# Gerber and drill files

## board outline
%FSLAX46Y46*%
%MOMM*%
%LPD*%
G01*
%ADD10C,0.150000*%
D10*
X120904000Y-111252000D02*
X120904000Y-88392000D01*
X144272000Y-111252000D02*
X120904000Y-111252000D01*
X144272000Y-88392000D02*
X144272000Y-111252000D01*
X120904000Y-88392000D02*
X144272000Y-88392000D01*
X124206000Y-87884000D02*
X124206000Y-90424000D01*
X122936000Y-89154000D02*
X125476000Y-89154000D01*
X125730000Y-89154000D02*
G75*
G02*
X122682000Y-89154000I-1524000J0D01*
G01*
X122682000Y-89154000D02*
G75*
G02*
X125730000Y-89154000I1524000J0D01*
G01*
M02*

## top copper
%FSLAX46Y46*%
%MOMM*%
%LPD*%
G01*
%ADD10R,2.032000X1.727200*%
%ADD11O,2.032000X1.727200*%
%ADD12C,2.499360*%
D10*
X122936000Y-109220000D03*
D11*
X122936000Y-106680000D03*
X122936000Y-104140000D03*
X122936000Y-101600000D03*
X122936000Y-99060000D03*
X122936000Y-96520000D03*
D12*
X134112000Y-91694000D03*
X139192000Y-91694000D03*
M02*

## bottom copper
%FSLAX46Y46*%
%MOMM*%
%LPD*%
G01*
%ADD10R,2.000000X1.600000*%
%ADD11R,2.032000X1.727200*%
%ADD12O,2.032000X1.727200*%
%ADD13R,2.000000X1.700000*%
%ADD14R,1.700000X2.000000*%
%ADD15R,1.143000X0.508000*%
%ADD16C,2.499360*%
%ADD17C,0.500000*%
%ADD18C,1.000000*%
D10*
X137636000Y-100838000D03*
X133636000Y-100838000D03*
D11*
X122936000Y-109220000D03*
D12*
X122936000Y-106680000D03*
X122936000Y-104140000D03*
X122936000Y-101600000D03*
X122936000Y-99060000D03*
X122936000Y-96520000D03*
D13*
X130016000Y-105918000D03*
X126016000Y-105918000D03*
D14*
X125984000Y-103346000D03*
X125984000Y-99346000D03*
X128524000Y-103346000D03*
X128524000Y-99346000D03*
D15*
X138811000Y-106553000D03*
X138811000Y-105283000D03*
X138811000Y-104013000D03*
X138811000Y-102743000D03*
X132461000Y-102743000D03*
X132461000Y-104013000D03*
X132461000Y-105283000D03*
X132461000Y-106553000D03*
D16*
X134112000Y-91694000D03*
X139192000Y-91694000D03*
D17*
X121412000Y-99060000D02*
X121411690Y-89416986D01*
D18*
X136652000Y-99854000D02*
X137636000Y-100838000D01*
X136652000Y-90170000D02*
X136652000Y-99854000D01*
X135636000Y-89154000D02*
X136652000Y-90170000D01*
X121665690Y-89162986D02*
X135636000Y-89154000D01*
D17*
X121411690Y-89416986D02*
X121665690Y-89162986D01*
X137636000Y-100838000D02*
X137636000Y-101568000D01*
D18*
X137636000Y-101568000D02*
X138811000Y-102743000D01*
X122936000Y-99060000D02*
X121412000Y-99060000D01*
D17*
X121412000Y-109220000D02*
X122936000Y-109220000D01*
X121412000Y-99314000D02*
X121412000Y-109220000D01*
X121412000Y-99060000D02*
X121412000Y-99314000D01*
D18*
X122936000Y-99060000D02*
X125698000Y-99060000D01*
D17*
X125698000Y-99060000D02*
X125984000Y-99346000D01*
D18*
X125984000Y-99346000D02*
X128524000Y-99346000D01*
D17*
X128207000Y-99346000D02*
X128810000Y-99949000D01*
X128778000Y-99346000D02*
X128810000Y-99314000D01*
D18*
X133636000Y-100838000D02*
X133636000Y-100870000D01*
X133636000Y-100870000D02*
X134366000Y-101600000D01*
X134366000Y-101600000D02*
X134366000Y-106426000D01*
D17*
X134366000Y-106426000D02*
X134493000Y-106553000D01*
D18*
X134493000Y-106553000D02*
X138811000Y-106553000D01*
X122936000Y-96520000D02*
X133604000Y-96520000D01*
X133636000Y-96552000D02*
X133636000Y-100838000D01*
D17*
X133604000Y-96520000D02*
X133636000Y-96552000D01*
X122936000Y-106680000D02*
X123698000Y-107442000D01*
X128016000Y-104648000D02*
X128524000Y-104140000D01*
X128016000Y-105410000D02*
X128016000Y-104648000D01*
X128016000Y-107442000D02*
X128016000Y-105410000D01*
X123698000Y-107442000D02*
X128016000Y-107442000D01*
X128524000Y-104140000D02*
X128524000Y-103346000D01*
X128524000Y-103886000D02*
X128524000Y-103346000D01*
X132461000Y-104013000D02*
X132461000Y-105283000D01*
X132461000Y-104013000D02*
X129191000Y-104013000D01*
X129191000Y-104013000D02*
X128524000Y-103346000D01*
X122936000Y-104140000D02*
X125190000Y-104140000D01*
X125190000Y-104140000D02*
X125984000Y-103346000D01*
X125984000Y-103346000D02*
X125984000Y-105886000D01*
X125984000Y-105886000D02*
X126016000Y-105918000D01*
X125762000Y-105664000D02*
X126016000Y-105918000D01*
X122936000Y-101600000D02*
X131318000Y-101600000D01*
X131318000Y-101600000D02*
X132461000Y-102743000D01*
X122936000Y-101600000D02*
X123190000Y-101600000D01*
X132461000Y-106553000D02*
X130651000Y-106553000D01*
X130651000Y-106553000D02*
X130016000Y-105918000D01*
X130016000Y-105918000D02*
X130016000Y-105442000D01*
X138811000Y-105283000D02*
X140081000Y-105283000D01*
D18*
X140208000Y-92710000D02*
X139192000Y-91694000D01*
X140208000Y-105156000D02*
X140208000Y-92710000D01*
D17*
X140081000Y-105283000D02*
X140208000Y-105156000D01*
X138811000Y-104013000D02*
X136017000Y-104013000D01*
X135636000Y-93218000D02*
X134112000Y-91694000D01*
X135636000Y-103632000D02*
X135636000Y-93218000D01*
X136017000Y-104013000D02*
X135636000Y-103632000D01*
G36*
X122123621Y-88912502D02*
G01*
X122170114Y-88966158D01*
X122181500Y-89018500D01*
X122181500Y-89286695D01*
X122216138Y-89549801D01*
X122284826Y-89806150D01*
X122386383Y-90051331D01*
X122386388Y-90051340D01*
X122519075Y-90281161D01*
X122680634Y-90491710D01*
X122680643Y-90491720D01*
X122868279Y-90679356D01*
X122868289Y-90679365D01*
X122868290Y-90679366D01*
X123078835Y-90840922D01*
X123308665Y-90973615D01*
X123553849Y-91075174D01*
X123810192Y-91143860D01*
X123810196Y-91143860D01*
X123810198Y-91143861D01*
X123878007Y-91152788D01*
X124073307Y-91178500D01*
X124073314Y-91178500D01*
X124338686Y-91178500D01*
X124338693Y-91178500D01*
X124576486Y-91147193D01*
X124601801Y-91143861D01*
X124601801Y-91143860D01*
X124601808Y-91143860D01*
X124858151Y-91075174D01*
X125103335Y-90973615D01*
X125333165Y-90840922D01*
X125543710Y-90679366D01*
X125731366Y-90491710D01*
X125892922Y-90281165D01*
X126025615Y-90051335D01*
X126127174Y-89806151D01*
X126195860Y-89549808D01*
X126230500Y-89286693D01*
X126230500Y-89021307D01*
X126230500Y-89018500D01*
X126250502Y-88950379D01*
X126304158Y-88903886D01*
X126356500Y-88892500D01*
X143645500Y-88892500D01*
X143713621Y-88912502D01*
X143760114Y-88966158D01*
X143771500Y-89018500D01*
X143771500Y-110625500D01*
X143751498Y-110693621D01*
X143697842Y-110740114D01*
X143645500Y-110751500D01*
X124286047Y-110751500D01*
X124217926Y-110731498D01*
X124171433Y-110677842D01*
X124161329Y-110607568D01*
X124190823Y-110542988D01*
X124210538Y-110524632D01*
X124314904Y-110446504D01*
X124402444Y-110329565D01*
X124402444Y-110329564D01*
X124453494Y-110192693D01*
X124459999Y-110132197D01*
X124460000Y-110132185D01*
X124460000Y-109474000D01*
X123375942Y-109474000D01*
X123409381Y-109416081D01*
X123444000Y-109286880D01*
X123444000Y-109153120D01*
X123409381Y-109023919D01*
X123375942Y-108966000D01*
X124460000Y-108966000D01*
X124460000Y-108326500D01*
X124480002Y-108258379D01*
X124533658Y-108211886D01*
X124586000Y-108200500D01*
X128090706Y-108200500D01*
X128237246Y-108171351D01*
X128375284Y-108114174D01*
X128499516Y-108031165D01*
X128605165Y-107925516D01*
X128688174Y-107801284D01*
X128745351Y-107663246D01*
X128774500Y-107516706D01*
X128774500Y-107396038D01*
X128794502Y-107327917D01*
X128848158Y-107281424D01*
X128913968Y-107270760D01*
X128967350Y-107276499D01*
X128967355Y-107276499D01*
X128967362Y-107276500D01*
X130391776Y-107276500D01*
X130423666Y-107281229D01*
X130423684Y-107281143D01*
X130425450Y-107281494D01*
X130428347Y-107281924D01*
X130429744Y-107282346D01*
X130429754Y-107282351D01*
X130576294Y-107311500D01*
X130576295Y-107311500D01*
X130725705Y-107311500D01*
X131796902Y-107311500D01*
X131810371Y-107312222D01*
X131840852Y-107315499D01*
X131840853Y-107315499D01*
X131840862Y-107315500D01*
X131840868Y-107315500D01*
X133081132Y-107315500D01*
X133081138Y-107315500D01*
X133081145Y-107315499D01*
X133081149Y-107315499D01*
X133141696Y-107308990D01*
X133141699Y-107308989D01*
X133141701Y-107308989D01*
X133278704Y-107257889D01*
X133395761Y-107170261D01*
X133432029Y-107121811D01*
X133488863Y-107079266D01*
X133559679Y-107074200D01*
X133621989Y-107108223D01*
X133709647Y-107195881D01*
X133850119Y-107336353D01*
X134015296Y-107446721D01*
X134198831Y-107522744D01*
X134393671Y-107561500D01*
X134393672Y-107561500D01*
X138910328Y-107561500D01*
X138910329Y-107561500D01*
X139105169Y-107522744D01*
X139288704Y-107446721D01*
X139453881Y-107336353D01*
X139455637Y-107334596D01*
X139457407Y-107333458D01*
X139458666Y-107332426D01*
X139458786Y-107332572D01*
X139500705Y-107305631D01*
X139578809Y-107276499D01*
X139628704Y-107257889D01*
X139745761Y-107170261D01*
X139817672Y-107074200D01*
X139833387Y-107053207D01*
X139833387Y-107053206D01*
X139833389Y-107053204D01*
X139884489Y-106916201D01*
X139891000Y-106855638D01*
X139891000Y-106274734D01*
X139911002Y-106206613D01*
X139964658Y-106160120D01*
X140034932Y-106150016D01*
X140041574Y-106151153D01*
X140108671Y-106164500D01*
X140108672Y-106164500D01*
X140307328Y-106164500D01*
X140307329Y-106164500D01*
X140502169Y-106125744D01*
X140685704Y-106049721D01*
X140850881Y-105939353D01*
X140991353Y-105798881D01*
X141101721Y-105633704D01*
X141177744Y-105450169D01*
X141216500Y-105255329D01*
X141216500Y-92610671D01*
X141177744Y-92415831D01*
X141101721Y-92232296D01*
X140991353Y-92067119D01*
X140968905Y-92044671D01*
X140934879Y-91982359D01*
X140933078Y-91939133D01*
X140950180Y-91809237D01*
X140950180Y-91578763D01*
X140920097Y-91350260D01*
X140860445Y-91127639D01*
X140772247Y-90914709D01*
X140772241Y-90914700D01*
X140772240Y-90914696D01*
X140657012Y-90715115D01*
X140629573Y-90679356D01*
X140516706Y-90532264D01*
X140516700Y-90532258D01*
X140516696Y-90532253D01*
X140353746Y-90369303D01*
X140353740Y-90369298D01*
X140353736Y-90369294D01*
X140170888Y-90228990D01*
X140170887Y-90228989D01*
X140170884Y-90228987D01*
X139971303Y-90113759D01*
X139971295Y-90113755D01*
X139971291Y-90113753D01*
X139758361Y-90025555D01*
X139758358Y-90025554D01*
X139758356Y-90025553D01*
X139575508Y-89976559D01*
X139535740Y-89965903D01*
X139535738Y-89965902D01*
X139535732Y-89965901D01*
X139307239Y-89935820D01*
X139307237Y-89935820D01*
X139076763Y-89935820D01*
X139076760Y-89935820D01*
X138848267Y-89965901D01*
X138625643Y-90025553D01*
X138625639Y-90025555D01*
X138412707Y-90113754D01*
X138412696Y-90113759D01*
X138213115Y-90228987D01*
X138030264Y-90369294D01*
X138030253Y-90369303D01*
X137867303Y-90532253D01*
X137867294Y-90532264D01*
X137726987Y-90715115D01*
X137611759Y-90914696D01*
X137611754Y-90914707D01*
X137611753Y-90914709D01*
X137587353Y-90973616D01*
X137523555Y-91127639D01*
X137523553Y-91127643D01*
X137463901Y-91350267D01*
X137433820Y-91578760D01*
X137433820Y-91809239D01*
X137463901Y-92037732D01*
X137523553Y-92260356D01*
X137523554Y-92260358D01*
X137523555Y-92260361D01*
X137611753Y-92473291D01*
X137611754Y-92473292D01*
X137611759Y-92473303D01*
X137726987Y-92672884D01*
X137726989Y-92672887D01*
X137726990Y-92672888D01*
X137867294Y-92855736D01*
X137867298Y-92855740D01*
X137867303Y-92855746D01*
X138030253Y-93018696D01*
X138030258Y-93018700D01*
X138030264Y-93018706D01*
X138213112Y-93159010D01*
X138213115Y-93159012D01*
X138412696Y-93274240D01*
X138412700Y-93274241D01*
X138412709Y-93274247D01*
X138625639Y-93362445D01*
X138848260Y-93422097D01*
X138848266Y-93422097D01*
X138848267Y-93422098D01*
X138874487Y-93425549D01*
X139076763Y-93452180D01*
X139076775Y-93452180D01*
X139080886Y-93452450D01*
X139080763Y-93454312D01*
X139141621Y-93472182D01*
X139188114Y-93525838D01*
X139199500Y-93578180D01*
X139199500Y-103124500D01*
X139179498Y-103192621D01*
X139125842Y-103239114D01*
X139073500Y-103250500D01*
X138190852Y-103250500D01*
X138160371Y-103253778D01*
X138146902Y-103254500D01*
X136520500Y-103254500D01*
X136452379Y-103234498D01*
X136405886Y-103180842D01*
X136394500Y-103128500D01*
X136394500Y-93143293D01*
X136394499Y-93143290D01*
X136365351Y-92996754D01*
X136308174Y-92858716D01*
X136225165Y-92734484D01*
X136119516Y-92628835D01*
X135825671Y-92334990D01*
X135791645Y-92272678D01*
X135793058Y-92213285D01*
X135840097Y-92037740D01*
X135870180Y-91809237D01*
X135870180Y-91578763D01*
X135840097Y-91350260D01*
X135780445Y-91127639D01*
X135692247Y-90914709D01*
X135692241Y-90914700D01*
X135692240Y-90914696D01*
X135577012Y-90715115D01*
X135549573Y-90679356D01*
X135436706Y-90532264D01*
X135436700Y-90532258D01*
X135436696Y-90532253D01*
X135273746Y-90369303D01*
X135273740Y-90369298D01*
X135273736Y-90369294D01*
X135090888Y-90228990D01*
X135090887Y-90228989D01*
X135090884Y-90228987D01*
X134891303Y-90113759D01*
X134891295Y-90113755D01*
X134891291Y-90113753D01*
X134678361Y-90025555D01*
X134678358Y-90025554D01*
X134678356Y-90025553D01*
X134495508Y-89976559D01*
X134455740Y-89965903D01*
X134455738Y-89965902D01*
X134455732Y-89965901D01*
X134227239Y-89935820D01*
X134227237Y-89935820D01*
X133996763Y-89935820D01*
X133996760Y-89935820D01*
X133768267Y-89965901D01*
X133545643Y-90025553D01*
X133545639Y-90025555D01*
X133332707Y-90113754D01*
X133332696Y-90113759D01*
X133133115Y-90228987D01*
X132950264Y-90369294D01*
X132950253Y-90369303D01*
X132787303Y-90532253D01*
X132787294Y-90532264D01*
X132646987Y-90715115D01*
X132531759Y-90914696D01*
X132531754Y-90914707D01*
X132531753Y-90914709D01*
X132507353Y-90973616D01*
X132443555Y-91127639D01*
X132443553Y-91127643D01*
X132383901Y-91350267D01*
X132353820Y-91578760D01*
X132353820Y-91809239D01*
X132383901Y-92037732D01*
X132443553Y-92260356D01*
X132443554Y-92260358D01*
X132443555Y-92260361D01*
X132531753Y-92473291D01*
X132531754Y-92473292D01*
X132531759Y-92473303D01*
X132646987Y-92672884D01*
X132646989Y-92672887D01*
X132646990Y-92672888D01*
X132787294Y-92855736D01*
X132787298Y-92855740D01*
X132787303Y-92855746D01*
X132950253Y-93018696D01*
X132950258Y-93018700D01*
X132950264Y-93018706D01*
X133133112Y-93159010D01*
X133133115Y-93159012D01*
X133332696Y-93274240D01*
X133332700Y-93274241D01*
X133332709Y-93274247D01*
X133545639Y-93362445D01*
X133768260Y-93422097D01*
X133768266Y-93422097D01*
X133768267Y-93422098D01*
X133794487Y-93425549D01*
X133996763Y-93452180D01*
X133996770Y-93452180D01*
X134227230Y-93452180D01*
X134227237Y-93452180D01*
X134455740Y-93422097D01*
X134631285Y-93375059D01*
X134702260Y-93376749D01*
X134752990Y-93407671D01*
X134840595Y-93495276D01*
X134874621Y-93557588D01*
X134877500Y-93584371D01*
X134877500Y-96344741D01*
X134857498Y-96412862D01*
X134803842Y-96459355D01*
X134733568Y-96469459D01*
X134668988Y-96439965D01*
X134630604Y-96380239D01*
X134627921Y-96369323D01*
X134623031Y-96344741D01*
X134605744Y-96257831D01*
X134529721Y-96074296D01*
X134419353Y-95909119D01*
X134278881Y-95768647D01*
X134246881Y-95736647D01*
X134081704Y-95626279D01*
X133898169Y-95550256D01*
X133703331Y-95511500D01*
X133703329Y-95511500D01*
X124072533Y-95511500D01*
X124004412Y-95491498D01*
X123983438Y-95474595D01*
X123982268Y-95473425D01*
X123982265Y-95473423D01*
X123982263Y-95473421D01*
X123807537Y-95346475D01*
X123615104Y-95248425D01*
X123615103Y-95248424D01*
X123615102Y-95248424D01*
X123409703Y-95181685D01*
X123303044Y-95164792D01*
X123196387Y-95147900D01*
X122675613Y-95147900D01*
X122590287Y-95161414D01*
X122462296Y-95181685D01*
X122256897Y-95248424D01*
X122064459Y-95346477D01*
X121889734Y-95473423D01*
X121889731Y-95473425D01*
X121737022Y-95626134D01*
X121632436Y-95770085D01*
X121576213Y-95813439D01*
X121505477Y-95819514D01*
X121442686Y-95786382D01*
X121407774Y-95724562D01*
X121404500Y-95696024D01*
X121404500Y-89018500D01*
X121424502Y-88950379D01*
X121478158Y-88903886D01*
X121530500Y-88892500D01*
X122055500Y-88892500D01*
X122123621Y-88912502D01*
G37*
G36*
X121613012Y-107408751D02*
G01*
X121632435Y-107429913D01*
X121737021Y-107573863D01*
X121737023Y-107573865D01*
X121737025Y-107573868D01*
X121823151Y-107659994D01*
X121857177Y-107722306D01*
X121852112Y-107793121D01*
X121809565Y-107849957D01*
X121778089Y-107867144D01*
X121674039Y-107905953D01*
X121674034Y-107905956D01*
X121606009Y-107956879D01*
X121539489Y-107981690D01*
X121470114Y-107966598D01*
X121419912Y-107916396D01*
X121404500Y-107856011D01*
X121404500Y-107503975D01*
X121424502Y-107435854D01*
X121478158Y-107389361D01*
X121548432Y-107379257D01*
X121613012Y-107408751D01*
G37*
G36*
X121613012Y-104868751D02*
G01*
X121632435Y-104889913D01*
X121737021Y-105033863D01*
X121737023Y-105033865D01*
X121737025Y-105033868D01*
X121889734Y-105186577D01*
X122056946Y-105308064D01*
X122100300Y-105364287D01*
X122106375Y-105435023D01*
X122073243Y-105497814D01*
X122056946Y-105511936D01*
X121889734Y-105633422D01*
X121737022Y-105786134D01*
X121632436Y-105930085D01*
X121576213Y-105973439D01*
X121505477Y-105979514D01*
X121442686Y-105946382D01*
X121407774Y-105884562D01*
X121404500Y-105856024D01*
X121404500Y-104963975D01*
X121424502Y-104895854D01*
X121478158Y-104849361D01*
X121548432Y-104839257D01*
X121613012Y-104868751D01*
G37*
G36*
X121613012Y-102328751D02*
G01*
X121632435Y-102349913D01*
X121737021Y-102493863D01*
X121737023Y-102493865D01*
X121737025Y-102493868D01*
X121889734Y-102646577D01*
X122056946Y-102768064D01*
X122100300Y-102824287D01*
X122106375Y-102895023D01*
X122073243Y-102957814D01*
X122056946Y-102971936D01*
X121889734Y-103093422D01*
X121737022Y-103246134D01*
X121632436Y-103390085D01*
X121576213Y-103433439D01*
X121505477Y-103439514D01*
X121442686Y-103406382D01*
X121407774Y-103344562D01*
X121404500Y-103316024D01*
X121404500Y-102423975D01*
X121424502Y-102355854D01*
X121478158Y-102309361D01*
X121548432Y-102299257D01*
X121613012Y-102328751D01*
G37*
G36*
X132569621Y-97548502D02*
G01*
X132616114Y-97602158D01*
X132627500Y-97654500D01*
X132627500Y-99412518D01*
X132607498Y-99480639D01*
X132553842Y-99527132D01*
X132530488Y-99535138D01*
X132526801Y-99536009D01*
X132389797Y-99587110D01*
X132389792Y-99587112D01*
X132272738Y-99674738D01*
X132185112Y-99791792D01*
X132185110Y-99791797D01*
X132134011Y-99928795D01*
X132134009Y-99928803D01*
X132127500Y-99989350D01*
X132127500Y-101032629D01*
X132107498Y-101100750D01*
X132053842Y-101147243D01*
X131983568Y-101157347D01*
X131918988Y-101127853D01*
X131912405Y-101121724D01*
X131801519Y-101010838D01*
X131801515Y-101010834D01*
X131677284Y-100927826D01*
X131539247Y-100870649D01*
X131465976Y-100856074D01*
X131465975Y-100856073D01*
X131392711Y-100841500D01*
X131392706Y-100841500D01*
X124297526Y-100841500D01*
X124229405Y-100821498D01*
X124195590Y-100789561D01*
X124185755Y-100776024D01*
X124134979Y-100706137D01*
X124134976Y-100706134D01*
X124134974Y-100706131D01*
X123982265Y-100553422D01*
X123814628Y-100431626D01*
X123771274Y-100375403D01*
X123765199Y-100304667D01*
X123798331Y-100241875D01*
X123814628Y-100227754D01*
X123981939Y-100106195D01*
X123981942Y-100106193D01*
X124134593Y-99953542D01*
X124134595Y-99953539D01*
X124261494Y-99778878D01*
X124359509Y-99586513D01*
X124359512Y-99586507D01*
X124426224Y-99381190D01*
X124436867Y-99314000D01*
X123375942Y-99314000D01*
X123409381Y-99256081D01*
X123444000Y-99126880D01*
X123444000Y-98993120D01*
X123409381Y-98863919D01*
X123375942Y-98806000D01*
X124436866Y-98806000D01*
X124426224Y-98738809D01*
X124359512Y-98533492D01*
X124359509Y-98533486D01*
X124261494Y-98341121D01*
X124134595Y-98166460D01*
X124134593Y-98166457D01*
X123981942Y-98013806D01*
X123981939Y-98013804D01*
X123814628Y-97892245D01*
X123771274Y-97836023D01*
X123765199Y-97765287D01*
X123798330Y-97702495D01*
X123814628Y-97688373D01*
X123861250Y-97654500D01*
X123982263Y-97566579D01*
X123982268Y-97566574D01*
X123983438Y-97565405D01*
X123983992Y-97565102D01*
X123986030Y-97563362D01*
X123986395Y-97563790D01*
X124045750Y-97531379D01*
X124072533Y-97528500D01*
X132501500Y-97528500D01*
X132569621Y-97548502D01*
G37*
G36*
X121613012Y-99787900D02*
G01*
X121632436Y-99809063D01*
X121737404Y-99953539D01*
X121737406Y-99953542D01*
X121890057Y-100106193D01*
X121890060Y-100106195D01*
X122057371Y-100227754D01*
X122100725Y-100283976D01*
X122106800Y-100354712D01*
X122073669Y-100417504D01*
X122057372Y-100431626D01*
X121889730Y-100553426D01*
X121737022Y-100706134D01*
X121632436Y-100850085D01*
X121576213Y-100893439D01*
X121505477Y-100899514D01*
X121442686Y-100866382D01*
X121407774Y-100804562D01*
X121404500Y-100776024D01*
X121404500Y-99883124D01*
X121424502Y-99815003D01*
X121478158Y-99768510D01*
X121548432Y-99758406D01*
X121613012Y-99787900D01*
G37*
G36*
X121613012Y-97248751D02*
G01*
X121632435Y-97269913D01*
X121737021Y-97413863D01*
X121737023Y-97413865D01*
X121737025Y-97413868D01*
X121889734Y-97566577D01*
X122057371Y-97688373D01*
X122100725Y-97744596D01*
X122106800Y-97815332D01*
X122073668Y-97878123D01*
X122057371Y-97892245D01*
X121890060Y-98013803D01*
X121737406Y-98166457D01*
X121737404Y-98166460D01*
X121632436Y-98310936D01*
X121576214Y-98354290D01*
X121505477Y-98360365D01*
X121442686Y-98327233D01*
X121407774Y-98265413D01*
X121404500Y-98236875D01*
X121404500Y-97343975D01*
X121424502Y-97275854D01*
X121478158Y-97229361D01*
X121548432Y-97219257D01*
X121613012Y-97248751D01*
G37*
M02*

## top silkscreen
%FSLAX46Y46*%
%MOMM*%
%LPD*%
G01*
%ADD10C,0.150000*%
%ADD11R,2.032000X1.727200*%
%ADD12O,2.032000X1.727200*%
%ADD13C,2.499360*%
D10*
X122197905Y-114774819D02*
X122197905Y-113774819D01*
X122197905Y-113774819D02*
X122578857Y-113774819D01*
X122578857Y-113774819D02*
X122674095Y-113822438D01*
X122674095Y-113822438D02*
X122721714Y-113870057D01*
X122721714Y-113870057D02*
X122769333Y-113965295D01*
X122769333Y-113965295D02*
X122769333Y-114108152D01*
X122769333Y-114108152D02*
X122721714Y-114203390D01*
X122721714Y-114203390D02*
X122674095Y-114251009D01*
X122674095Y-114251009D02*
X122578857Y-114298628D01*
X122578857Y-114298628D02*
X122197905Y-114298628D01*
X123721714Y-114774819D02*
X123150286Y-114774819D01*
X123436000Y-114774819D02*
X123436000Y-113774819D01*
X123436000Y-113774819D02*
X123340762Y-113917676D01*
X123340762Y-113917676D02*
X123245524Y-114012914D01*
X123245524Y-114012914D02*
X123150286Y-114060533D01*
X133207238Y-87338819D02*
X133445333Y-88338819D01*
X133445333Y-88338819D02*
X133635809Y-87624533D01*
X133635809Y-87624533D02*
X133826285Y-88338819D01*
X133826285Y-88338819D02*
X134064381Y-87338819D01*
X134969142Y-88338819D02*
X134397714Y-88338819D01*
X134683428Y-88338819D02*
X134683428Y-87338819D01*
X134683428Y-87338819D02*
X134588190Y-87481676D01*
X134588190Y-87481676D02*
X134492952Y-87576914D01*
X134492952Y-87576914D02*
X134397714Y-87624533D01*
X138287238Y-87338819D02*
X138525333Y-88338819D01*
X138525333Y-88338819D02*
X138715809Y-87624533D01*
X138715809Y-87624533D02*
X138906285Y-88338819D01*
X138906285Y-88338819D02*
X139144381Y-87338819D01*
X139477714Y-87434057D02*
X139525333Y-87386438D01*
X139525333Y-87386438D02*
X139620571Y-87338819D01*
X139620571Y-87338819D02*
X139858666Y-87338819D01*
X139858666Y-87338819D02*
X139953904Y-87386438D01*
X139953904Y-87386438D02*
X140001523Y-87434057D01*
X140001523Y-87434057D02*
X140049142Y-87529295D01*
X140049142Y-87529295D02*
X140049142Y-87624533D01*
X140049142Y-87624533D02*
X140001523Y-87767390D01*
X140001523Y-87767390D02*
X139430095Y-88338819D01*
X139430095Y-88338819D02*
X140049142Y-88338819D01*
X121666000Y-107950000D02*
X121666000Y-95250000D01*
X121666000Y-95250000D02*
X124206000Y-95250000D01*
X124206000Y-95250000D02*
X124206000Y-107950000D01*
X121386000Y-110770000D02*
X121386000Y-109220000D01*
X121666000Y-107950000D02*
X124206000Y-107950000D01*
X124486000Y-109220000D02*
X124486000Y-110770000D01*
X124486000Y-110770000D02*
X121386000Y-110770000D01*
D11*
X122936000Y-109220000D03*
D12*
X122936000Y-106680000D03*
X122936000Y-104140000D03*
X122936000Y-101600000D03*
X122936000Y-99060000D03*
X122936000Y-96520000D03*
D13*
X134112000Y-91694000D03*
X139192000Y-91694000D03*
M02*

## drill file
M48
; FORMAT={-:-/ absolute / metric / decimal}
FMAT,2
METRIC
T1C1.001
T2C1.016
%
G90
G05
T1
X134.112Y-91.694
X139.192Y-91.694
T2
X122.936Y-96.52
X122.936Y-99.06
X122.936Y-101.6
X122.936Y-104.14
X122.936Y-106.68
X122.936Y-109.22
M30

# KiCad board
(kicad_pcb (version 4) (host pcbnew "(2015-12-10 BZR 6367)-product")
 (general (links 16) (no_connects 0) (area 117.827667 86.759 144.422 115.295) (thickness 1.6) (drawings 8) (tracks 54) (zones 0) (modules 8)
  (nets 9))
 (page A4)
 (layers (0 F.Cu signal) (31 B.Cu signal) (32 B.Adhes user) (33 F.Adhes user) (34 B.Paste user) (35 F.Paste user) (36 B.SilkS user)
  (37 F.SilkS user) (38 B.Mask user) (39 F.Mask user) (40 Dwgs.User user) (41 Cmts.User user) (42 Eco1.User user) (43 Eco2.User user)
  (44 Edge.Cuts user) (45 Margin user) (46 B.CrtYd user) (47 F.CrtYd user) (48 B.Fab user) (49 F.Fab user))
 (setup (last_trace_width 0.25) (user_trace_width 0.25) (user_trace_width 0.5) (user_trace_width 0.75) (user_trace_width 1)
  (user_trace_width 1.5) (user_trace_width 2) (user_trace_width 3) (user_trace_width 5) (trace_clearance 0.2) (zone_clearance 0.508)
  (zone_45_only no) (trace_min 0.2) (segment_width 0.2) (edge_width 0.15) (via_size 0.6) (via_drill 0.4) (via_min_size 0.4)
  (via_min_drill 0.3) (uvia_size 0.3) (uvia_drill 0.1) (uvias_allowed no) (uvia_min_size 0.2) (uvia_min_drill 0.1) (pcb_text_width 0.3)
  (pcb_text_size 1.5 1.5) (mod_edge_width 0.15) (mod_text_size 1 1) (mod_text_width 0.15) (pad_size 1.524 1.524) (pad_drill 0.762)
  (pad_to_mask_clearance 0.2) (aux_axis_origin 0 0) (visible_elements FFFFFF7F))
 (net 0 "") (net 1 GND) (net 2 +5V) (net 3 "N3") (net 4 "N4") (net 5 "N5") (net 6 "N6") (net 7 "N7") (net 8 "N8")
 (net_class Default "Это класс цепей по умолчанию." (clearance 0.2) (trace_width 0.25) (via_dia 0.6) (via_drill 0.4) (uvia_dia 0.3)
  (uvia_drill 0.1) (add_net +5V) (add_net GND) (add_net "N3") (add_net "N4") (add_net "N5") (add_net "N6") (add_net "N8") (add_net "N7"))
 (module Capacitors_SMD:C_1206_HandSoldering (layer B.Cu) (at 135.636 100.838 180)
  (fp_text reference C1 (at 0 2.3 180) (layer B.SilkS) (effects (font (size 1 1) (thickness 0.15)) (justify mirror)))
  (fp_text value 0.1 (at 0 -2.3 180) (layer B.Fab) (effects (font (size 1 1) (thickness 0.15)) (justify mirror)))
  (pad 1 smd rect (at -2 0 180) (size 2 1.6) (layers B.Cu B.Paste B.Mask) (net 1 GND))
  (pad 2 smd rect (at 2 0 180) (size 2 1.6) (layers B.Cu B.Paste B.Mask) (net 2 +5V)))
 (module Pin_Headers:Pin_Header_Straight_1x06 (layer F.Cu) (at 122.936 109.22 180)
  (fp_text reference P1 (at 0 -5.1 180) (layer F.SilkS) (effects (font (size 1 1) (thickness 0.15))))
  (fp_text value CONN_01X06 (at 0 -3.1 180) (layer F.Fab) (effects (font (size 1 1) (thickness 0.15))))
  (fp_line (start 1.27 1.27) (end 1.27 13.97) (layer F.SilkS) (width 0.15))
  (fp_line (start 1.27 13.97) (end -1.27 13.97) (layer F.SilkS) (width 0.15))
  (fp_line (start -1.27 13.97) (end -1.27 1.27) (layer F.SilkS) (width 0.15))
  (fp_line (start 1.55 -1.55) (end 1.55 0) (layer F.SilkS) (width 0.15))
  (fp_line (start 1.27 1.27) (end -1.27 1.27) (layer F.SilkS) (width 0.15))
  (fp_line (start -1.55 0) (end -1.55 -1.55) (layer F.SilkS) (width 0.15))
  (fp_line (start -1.55 -1.55) (end 1.55 -1.55) (layer F.SilkS) (width 0.15))
  (pad 1 thru_hole rect (at 0 0 180) (size 2.032 1.7272) (drill 1.016) (layers *.Cu *.Mask F.SilkS) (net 1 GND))
  (pad 2 thru_hole oval (at 0 2.54 180) (size 2.032 1.7272) (drill 1.016) (layers *.Cu *.Mask F.SilkS) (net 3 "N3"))
  (pad 3 thru_hole oval (at 0 5.08 180) (size 2.032 1.7272) (drill 1.016) (layers *.Cu *.Mask F.SilkS) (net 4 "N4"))
  (pad 4 thru_hole oval (at 0 7.62 180) (size 2.032 1.7272) (drill 1.016) (layers *.Cu *.Mask F.SilkS) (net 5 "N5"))
  (pad 5 thru_hole oval (at 0 10.16 180) (size 2.032 1.7272) (drill 1.016) (layers *.Cu *.Mask F.SilkS) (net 1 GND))
  (pad 6 thru_hole oval (at 0 12.7 180) (size 2.032 1.7272) (drill 1.016) (layers *.Cu *.Mask F.SilkS) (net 2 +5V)))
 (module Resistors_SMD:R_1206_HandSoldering (layer B.Cu) (at 128.016 105.918 180)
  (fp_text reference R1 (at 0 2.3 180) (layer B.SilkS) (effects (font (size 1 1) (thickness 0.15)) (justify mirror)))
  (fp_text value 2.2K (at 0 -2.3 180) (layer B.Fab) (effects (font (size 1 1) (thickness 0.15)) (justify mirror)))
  (pad 1 smd rect (at -2 0 180) (size 2 1.7) (layers B.Cu B.Paste B.Mask) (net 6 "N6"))
  (pad 2 smd rect (at 2 0 180) (size 2 1.7) (layers B.Cu B.Paste B.Mask) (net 4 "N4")))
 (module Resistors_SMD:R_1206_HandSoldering (layer B.Cu) (at 125.984 101.346 90)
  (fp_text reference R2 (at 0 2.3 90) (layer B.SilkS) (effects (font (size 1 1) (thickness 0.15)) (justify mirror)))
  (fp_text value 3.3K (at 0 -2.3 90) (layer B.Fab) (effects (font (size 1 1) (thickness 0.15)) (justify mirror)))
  (pad 1 smd rect (at -2 0 90) (size 2 1.7) (layers B.Cu B.Paste B.Mask) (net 4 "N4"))
  (pad 2 smd rect (at 2 0 90) (size 2 1.7) (layers B.Cu B.Paste B.Mask) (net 1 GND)))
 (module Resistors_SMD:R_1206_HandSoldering (layer B.Cu) (at 128.524 101.346 90)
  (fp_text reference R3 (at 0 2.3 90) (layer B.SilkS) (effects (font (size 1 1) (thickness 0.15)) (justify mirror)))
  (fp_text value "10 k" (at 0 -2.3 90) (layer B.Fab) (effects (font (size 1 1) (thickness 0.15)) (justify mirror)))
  (pad 1 smd rect (at -2 0 90) (size 2 1.7) (layers B.Cu B.Paste B.Mask) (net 3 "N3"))
  (pad 2 smd rect (at 2 0 90) (size 2 1.7) (layers B.Cu B.Paste B.Mask) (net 1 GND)))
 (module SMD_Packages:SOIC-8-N (layer B.Cu) (at 135.636 104.648 90)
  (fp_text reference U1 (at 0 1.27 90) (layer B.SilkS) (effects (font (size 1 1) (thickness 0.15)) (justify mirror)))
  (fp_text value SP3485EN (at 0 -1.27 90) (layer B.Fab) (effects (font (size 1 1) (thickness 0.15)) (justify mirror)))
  (pad 8 smd rect (at -1.905 3.175 90) (size 0.508 1.143) (layers B.Cu B.Paste B.Mask) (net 2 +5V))
  (pad 7 smd rect (at -0.635 3.175 90) (size 0.508 1.143) (layers B.Cu B.Paste B.Mask) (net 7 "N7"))
  (pad 6 smd rect (at 0.635 3.175 90) (size 0.508 1.143) (layers B.Cu B.Paste B.Mask) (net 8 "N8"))
  (pad 5 smd rect (at 1.905 3.175 90) (size 0.508 1.143) (layers B.Cu B.Paste B.Mask) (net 1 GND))
  (pad 4 smd rect (at 1.905 -3.175 90) (size 0.508 1.143) (layers B.Cu B.Paste B.Mask) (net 5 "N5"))
  (pad 3 smd rect (at 0.635 -3.175 90) (size 0.508 1.143) (layers B.Cu B.Paste B.Mask) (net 3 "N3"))
  (pad 2 smd rect (at -0.635 -3.175 90) (size 0.508 1.143) (layers B.Cu B.Paste B.Mask) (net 3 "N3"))
  (pad 1 smd rect (at -1.905 -3.175 90) (size 0.508 1.143) (layers B.Cu B.Paste B.Mask) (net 6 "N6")))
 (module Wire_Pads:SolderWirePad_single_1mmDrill (layer F.Cu) (at 134.112 91.694)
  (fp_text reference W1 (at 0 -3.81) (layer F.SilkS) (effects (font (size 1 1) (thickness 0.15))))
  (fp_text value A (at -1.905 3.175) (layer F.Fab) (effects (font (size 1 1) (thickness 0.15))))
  (pad 1 thru_hole circle (at 0 0) (size 2.49936 2.49936) (drill 1.00076) (layers *.Cu *.Mask F.SilkS) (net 8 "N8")))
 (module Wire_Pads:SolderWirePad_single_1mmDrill (layer F.Cu) (at 139.192 91.694)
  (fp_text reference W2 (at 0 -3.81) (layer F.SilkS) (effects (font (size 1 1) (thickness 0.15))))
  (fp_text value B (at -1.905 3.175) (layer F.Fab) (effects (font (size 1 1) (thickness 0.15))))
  (pad 1 thru_hole circle (at 0 0) (size 2.49936 2.49936) (drill 1.00076) (layers *.Cu *.Mask F.SilkS) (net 7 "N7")))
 (gr_line (start 120.904 111.252) (end 120.904 88.392) (angle 90) (layer Edge.Cuts) (width 0.15))
 (gr_line (start 144.272 111.252) (end 120.904 111.252) (angle 90) (layer Edge.Cuts) (width 0.15))
 (gr_line (start 144.272 88.392) (end 144.272 111.252) (angle 90) (layer Edge.Cuts) (width 0.15))
 (gr_line (start 120.904 88.392) (end 144.272 88.392) (angle 90) (layer Edge.Cuts) (width 0.15))
 (gr_line (start 124.206 87.884) (end 124.206 90.424) (angle 90) (layer Edge.Cuts) (width 0.15))
 (gr_line (start 122.936 89.154) (end 125.476 89.154) (angle 90) (layer Edge.Cuts) (width 0.15))
 (gr_circle (center 124.206 89.154) (end 125.73 89.154) (layer Edge.Cuts) (width 0.15))
 (segment (start 121.412 99.06) (end 121.41169 89.416986) (width 0.5) (layer B.Cu) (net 1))
 (segment (start 136.652 99.854) (end 137.636 100.838) (width 1) (layer B.Cu) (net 1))
 (segment (start 136.652 90.17) (end 136.652 99.854) (width 1) (layer B.Cu) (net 1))
 (segment (start 135.636 89.154) (end 136.652 90.17) (width 1) (layer B.Cu) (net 1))
 (segment (start 121.66569 89.162986) (end 135.636 89.154) (width 1) (layer B.Cu) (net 1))
 (segment (start 121.41169 89.416986) (end 121.66569 89.162986) (width 0.5) (layer B.Cu) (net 1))
 (segment (start 137.636 100.838) (end 137.636 101.568) (width 0.5) (layer B.Cu) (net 1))
 (segment (start 137.636 101.568) (end 138.811 102.743) (width 1) (layer B.Cu) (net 1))
 (segment (start 122.936 99.06) (end 121.412 99.06) (width 1) (layer B.Cu) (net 1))
 (segment (start 121.412 109.22) (end 122.936 109.22) (width 0.5) (layer B.Cu) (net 1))
 (segment (start 121.412 99.314) (end 121.412 109.22) (width 0.5) (layer B.Cu) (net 1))
 (segment (start 121.412 99.06) (end 121.412 99.314) (width 0.5) (layer B.Cu) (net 1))
 (segment (start 122.936 99.06) (end 125.698 99.06) (width 1) (layer B.Cu) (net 1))
 (segment (start 125.698 99.06) (end 125.984 99.346) (width 0.5) (layer B.Cu) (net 1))
 (segment (start 125.984 99.346) (end 128.524 99.346) (width 1) (layer B.Cu) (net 1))
 (segment (start 128.207 99.346) (end 128.81 99.949) (width 0.5) (layer B.Cu) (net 1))
 (segment (start 128.778 99.346) (end 128.81 99.314) (width 0.5) (layer B.Cu) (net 1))
 (segment (start 133.636 100.838) (end 133.636 100.87) (width 1) (layer B.Cu) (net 2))
 (segment (start 133.636 100.87) (end 134.366 101.6) (width 1) (layer B.Cu) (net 2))
 (segment (start 134.366 101.6) (end 134.366 106.426) (width 1) (layer B.Cu) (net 2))
 (segment (start 134.366 106.426) (end 134.493 106.553) (width 0.5) (layer B.Cu) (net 2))
 (segment (start 134.493 106.553) (end 138.811 106.553) (width 1) (layer B.Cu) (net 2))
 (segment (start 122.936 96.52) (end 133.604 96.52) (width 1) (layer B.Cu) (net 2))
 (segment (start 133.636 96.552) (end 133.636 100.838) (width 1) (layer B.Cu) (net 2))
 (segment (start 133.604 96.52) (end 133.636 96.552) (width 0.5) (layer B.Cu) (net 2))
 (segment (start 122.936 106.68) (end 123.698 107.442) (width 0.5) (layer B.Cu) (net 3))
 (segment (start 128.016 104.648) (end 128.524 104.14) (width 0.5) (layer B.Cu) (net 3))
 (segment (start 128.016 105.41) (end 128.016 104.648) (width 0.5) (layer B.Cu) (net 3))
 (segment (start 128.016 107.442) (end 128.016 105.41) (width 0.5) (layer B.Cu) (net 3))
 (segment (start 123.698 107.442) (end 128.016 107.442) (width 0.5) (layer B.Cu) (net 3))
 (segment (start 128.524 104.14) (end 128.524 103.346) (width 0.5) (layer B.Cu) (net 3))
 (segment (start 128.524 103.886) (end 128.524 103.346) (width 0.5) (layer B.Cu) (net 3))
 (segment (start 132.461 104.013) (end 132.461 105.283) (width 0.5) (layer B.Cu) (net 3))
 (segment (start 132.461 104.013) (end 129.191 104.013) (width 0.5) (layer B.Cu) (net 3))
 (segment (start 129.191 104.013) (end 128.524 103.346) (width 0.5) (layer B.Cu) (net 3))
 (segment (start 122.936 104.14) (end 125.19 104.14) (width 0.5) (layer B.Cu) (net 4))
 (segment (start 125.19 104.14) (end 125.984 103.346) (width 0.5) (layer B.Cu) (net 4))
 (segment (start 125.984 103.346) (end 125.984 105.886) (width 0.5) (layer B.Cu) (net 4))
 (segment (start 125.984 105.886) (end 126.016 105.918) (width 0.5) (layer B.Cu) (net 4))
 (segment (start 125.762 105.664) (end 126.016 105.918) (width 0.5) (layer B.Cu) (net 4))
 (segment (start 122.936 101.6) (end 131.318 101.6) (width 0.5) (layer B.Cu) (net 5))
 (segment (start 131.318 101.6) (end 132.461 102.743) (width 0.5) (layer B.Cu) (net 5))
 (segment (start 122.936 101.6) (end 123.19 101.6) (width 0.5) (layer B.Cu) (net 5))
 (segment (start 132.461 106.553) (end 130.651 106.553) (width 0.5) (layer B.Cu) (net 6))
 (segment (start 130.651 106.553) (end 130.016 105.918) (width 0.5) (layer B.Cu) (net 6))
 (segment (start 130.016 105.918) (end 130.016 105.442) (width 0.5) (layer B.Cu) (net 6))
 (segment (start 138.811 105.283) (end 140.081 105.283) (width 0.5) (layer B.Cu) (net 7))
 (segment (start 140.208 92.71) (end 139.192 91.694) (width 1) (layer B.Cu) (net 7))
 (segment (start 140.208 105.156) (end 140.208 92.71) (width 1) (layer B.Cu) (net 7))
 (segment (start 140.081 105.283) (end 140.208 105.156) (width 0.5) (layer B.Cu) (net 7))
 (segment (start 138.811 104.013) (end 136.017 104.013) (width 0.5) (layer B.Cu) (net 8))
 (segment (start 135.636 93.218) (end 134.112 91.694) (width 0.5) (layer B.Cu) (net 8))
 (segment (start 135.636 103.632) (end 135.636 93.218) (width 0.5) (layer B.Cu) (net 8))
 (segment (start 136.017 104.013) (end 135.636 103.632) (width 0.5) (layer B.Cu) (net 8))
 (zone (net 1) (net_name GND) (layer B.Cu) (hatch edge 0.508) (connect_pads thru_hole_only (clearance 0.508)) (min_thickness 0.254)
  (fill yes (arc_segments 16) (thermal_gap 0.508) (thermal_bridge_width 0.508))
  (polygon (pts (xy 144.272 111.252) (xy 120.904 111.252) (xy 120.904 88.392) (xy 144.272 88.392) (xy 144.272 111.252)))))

